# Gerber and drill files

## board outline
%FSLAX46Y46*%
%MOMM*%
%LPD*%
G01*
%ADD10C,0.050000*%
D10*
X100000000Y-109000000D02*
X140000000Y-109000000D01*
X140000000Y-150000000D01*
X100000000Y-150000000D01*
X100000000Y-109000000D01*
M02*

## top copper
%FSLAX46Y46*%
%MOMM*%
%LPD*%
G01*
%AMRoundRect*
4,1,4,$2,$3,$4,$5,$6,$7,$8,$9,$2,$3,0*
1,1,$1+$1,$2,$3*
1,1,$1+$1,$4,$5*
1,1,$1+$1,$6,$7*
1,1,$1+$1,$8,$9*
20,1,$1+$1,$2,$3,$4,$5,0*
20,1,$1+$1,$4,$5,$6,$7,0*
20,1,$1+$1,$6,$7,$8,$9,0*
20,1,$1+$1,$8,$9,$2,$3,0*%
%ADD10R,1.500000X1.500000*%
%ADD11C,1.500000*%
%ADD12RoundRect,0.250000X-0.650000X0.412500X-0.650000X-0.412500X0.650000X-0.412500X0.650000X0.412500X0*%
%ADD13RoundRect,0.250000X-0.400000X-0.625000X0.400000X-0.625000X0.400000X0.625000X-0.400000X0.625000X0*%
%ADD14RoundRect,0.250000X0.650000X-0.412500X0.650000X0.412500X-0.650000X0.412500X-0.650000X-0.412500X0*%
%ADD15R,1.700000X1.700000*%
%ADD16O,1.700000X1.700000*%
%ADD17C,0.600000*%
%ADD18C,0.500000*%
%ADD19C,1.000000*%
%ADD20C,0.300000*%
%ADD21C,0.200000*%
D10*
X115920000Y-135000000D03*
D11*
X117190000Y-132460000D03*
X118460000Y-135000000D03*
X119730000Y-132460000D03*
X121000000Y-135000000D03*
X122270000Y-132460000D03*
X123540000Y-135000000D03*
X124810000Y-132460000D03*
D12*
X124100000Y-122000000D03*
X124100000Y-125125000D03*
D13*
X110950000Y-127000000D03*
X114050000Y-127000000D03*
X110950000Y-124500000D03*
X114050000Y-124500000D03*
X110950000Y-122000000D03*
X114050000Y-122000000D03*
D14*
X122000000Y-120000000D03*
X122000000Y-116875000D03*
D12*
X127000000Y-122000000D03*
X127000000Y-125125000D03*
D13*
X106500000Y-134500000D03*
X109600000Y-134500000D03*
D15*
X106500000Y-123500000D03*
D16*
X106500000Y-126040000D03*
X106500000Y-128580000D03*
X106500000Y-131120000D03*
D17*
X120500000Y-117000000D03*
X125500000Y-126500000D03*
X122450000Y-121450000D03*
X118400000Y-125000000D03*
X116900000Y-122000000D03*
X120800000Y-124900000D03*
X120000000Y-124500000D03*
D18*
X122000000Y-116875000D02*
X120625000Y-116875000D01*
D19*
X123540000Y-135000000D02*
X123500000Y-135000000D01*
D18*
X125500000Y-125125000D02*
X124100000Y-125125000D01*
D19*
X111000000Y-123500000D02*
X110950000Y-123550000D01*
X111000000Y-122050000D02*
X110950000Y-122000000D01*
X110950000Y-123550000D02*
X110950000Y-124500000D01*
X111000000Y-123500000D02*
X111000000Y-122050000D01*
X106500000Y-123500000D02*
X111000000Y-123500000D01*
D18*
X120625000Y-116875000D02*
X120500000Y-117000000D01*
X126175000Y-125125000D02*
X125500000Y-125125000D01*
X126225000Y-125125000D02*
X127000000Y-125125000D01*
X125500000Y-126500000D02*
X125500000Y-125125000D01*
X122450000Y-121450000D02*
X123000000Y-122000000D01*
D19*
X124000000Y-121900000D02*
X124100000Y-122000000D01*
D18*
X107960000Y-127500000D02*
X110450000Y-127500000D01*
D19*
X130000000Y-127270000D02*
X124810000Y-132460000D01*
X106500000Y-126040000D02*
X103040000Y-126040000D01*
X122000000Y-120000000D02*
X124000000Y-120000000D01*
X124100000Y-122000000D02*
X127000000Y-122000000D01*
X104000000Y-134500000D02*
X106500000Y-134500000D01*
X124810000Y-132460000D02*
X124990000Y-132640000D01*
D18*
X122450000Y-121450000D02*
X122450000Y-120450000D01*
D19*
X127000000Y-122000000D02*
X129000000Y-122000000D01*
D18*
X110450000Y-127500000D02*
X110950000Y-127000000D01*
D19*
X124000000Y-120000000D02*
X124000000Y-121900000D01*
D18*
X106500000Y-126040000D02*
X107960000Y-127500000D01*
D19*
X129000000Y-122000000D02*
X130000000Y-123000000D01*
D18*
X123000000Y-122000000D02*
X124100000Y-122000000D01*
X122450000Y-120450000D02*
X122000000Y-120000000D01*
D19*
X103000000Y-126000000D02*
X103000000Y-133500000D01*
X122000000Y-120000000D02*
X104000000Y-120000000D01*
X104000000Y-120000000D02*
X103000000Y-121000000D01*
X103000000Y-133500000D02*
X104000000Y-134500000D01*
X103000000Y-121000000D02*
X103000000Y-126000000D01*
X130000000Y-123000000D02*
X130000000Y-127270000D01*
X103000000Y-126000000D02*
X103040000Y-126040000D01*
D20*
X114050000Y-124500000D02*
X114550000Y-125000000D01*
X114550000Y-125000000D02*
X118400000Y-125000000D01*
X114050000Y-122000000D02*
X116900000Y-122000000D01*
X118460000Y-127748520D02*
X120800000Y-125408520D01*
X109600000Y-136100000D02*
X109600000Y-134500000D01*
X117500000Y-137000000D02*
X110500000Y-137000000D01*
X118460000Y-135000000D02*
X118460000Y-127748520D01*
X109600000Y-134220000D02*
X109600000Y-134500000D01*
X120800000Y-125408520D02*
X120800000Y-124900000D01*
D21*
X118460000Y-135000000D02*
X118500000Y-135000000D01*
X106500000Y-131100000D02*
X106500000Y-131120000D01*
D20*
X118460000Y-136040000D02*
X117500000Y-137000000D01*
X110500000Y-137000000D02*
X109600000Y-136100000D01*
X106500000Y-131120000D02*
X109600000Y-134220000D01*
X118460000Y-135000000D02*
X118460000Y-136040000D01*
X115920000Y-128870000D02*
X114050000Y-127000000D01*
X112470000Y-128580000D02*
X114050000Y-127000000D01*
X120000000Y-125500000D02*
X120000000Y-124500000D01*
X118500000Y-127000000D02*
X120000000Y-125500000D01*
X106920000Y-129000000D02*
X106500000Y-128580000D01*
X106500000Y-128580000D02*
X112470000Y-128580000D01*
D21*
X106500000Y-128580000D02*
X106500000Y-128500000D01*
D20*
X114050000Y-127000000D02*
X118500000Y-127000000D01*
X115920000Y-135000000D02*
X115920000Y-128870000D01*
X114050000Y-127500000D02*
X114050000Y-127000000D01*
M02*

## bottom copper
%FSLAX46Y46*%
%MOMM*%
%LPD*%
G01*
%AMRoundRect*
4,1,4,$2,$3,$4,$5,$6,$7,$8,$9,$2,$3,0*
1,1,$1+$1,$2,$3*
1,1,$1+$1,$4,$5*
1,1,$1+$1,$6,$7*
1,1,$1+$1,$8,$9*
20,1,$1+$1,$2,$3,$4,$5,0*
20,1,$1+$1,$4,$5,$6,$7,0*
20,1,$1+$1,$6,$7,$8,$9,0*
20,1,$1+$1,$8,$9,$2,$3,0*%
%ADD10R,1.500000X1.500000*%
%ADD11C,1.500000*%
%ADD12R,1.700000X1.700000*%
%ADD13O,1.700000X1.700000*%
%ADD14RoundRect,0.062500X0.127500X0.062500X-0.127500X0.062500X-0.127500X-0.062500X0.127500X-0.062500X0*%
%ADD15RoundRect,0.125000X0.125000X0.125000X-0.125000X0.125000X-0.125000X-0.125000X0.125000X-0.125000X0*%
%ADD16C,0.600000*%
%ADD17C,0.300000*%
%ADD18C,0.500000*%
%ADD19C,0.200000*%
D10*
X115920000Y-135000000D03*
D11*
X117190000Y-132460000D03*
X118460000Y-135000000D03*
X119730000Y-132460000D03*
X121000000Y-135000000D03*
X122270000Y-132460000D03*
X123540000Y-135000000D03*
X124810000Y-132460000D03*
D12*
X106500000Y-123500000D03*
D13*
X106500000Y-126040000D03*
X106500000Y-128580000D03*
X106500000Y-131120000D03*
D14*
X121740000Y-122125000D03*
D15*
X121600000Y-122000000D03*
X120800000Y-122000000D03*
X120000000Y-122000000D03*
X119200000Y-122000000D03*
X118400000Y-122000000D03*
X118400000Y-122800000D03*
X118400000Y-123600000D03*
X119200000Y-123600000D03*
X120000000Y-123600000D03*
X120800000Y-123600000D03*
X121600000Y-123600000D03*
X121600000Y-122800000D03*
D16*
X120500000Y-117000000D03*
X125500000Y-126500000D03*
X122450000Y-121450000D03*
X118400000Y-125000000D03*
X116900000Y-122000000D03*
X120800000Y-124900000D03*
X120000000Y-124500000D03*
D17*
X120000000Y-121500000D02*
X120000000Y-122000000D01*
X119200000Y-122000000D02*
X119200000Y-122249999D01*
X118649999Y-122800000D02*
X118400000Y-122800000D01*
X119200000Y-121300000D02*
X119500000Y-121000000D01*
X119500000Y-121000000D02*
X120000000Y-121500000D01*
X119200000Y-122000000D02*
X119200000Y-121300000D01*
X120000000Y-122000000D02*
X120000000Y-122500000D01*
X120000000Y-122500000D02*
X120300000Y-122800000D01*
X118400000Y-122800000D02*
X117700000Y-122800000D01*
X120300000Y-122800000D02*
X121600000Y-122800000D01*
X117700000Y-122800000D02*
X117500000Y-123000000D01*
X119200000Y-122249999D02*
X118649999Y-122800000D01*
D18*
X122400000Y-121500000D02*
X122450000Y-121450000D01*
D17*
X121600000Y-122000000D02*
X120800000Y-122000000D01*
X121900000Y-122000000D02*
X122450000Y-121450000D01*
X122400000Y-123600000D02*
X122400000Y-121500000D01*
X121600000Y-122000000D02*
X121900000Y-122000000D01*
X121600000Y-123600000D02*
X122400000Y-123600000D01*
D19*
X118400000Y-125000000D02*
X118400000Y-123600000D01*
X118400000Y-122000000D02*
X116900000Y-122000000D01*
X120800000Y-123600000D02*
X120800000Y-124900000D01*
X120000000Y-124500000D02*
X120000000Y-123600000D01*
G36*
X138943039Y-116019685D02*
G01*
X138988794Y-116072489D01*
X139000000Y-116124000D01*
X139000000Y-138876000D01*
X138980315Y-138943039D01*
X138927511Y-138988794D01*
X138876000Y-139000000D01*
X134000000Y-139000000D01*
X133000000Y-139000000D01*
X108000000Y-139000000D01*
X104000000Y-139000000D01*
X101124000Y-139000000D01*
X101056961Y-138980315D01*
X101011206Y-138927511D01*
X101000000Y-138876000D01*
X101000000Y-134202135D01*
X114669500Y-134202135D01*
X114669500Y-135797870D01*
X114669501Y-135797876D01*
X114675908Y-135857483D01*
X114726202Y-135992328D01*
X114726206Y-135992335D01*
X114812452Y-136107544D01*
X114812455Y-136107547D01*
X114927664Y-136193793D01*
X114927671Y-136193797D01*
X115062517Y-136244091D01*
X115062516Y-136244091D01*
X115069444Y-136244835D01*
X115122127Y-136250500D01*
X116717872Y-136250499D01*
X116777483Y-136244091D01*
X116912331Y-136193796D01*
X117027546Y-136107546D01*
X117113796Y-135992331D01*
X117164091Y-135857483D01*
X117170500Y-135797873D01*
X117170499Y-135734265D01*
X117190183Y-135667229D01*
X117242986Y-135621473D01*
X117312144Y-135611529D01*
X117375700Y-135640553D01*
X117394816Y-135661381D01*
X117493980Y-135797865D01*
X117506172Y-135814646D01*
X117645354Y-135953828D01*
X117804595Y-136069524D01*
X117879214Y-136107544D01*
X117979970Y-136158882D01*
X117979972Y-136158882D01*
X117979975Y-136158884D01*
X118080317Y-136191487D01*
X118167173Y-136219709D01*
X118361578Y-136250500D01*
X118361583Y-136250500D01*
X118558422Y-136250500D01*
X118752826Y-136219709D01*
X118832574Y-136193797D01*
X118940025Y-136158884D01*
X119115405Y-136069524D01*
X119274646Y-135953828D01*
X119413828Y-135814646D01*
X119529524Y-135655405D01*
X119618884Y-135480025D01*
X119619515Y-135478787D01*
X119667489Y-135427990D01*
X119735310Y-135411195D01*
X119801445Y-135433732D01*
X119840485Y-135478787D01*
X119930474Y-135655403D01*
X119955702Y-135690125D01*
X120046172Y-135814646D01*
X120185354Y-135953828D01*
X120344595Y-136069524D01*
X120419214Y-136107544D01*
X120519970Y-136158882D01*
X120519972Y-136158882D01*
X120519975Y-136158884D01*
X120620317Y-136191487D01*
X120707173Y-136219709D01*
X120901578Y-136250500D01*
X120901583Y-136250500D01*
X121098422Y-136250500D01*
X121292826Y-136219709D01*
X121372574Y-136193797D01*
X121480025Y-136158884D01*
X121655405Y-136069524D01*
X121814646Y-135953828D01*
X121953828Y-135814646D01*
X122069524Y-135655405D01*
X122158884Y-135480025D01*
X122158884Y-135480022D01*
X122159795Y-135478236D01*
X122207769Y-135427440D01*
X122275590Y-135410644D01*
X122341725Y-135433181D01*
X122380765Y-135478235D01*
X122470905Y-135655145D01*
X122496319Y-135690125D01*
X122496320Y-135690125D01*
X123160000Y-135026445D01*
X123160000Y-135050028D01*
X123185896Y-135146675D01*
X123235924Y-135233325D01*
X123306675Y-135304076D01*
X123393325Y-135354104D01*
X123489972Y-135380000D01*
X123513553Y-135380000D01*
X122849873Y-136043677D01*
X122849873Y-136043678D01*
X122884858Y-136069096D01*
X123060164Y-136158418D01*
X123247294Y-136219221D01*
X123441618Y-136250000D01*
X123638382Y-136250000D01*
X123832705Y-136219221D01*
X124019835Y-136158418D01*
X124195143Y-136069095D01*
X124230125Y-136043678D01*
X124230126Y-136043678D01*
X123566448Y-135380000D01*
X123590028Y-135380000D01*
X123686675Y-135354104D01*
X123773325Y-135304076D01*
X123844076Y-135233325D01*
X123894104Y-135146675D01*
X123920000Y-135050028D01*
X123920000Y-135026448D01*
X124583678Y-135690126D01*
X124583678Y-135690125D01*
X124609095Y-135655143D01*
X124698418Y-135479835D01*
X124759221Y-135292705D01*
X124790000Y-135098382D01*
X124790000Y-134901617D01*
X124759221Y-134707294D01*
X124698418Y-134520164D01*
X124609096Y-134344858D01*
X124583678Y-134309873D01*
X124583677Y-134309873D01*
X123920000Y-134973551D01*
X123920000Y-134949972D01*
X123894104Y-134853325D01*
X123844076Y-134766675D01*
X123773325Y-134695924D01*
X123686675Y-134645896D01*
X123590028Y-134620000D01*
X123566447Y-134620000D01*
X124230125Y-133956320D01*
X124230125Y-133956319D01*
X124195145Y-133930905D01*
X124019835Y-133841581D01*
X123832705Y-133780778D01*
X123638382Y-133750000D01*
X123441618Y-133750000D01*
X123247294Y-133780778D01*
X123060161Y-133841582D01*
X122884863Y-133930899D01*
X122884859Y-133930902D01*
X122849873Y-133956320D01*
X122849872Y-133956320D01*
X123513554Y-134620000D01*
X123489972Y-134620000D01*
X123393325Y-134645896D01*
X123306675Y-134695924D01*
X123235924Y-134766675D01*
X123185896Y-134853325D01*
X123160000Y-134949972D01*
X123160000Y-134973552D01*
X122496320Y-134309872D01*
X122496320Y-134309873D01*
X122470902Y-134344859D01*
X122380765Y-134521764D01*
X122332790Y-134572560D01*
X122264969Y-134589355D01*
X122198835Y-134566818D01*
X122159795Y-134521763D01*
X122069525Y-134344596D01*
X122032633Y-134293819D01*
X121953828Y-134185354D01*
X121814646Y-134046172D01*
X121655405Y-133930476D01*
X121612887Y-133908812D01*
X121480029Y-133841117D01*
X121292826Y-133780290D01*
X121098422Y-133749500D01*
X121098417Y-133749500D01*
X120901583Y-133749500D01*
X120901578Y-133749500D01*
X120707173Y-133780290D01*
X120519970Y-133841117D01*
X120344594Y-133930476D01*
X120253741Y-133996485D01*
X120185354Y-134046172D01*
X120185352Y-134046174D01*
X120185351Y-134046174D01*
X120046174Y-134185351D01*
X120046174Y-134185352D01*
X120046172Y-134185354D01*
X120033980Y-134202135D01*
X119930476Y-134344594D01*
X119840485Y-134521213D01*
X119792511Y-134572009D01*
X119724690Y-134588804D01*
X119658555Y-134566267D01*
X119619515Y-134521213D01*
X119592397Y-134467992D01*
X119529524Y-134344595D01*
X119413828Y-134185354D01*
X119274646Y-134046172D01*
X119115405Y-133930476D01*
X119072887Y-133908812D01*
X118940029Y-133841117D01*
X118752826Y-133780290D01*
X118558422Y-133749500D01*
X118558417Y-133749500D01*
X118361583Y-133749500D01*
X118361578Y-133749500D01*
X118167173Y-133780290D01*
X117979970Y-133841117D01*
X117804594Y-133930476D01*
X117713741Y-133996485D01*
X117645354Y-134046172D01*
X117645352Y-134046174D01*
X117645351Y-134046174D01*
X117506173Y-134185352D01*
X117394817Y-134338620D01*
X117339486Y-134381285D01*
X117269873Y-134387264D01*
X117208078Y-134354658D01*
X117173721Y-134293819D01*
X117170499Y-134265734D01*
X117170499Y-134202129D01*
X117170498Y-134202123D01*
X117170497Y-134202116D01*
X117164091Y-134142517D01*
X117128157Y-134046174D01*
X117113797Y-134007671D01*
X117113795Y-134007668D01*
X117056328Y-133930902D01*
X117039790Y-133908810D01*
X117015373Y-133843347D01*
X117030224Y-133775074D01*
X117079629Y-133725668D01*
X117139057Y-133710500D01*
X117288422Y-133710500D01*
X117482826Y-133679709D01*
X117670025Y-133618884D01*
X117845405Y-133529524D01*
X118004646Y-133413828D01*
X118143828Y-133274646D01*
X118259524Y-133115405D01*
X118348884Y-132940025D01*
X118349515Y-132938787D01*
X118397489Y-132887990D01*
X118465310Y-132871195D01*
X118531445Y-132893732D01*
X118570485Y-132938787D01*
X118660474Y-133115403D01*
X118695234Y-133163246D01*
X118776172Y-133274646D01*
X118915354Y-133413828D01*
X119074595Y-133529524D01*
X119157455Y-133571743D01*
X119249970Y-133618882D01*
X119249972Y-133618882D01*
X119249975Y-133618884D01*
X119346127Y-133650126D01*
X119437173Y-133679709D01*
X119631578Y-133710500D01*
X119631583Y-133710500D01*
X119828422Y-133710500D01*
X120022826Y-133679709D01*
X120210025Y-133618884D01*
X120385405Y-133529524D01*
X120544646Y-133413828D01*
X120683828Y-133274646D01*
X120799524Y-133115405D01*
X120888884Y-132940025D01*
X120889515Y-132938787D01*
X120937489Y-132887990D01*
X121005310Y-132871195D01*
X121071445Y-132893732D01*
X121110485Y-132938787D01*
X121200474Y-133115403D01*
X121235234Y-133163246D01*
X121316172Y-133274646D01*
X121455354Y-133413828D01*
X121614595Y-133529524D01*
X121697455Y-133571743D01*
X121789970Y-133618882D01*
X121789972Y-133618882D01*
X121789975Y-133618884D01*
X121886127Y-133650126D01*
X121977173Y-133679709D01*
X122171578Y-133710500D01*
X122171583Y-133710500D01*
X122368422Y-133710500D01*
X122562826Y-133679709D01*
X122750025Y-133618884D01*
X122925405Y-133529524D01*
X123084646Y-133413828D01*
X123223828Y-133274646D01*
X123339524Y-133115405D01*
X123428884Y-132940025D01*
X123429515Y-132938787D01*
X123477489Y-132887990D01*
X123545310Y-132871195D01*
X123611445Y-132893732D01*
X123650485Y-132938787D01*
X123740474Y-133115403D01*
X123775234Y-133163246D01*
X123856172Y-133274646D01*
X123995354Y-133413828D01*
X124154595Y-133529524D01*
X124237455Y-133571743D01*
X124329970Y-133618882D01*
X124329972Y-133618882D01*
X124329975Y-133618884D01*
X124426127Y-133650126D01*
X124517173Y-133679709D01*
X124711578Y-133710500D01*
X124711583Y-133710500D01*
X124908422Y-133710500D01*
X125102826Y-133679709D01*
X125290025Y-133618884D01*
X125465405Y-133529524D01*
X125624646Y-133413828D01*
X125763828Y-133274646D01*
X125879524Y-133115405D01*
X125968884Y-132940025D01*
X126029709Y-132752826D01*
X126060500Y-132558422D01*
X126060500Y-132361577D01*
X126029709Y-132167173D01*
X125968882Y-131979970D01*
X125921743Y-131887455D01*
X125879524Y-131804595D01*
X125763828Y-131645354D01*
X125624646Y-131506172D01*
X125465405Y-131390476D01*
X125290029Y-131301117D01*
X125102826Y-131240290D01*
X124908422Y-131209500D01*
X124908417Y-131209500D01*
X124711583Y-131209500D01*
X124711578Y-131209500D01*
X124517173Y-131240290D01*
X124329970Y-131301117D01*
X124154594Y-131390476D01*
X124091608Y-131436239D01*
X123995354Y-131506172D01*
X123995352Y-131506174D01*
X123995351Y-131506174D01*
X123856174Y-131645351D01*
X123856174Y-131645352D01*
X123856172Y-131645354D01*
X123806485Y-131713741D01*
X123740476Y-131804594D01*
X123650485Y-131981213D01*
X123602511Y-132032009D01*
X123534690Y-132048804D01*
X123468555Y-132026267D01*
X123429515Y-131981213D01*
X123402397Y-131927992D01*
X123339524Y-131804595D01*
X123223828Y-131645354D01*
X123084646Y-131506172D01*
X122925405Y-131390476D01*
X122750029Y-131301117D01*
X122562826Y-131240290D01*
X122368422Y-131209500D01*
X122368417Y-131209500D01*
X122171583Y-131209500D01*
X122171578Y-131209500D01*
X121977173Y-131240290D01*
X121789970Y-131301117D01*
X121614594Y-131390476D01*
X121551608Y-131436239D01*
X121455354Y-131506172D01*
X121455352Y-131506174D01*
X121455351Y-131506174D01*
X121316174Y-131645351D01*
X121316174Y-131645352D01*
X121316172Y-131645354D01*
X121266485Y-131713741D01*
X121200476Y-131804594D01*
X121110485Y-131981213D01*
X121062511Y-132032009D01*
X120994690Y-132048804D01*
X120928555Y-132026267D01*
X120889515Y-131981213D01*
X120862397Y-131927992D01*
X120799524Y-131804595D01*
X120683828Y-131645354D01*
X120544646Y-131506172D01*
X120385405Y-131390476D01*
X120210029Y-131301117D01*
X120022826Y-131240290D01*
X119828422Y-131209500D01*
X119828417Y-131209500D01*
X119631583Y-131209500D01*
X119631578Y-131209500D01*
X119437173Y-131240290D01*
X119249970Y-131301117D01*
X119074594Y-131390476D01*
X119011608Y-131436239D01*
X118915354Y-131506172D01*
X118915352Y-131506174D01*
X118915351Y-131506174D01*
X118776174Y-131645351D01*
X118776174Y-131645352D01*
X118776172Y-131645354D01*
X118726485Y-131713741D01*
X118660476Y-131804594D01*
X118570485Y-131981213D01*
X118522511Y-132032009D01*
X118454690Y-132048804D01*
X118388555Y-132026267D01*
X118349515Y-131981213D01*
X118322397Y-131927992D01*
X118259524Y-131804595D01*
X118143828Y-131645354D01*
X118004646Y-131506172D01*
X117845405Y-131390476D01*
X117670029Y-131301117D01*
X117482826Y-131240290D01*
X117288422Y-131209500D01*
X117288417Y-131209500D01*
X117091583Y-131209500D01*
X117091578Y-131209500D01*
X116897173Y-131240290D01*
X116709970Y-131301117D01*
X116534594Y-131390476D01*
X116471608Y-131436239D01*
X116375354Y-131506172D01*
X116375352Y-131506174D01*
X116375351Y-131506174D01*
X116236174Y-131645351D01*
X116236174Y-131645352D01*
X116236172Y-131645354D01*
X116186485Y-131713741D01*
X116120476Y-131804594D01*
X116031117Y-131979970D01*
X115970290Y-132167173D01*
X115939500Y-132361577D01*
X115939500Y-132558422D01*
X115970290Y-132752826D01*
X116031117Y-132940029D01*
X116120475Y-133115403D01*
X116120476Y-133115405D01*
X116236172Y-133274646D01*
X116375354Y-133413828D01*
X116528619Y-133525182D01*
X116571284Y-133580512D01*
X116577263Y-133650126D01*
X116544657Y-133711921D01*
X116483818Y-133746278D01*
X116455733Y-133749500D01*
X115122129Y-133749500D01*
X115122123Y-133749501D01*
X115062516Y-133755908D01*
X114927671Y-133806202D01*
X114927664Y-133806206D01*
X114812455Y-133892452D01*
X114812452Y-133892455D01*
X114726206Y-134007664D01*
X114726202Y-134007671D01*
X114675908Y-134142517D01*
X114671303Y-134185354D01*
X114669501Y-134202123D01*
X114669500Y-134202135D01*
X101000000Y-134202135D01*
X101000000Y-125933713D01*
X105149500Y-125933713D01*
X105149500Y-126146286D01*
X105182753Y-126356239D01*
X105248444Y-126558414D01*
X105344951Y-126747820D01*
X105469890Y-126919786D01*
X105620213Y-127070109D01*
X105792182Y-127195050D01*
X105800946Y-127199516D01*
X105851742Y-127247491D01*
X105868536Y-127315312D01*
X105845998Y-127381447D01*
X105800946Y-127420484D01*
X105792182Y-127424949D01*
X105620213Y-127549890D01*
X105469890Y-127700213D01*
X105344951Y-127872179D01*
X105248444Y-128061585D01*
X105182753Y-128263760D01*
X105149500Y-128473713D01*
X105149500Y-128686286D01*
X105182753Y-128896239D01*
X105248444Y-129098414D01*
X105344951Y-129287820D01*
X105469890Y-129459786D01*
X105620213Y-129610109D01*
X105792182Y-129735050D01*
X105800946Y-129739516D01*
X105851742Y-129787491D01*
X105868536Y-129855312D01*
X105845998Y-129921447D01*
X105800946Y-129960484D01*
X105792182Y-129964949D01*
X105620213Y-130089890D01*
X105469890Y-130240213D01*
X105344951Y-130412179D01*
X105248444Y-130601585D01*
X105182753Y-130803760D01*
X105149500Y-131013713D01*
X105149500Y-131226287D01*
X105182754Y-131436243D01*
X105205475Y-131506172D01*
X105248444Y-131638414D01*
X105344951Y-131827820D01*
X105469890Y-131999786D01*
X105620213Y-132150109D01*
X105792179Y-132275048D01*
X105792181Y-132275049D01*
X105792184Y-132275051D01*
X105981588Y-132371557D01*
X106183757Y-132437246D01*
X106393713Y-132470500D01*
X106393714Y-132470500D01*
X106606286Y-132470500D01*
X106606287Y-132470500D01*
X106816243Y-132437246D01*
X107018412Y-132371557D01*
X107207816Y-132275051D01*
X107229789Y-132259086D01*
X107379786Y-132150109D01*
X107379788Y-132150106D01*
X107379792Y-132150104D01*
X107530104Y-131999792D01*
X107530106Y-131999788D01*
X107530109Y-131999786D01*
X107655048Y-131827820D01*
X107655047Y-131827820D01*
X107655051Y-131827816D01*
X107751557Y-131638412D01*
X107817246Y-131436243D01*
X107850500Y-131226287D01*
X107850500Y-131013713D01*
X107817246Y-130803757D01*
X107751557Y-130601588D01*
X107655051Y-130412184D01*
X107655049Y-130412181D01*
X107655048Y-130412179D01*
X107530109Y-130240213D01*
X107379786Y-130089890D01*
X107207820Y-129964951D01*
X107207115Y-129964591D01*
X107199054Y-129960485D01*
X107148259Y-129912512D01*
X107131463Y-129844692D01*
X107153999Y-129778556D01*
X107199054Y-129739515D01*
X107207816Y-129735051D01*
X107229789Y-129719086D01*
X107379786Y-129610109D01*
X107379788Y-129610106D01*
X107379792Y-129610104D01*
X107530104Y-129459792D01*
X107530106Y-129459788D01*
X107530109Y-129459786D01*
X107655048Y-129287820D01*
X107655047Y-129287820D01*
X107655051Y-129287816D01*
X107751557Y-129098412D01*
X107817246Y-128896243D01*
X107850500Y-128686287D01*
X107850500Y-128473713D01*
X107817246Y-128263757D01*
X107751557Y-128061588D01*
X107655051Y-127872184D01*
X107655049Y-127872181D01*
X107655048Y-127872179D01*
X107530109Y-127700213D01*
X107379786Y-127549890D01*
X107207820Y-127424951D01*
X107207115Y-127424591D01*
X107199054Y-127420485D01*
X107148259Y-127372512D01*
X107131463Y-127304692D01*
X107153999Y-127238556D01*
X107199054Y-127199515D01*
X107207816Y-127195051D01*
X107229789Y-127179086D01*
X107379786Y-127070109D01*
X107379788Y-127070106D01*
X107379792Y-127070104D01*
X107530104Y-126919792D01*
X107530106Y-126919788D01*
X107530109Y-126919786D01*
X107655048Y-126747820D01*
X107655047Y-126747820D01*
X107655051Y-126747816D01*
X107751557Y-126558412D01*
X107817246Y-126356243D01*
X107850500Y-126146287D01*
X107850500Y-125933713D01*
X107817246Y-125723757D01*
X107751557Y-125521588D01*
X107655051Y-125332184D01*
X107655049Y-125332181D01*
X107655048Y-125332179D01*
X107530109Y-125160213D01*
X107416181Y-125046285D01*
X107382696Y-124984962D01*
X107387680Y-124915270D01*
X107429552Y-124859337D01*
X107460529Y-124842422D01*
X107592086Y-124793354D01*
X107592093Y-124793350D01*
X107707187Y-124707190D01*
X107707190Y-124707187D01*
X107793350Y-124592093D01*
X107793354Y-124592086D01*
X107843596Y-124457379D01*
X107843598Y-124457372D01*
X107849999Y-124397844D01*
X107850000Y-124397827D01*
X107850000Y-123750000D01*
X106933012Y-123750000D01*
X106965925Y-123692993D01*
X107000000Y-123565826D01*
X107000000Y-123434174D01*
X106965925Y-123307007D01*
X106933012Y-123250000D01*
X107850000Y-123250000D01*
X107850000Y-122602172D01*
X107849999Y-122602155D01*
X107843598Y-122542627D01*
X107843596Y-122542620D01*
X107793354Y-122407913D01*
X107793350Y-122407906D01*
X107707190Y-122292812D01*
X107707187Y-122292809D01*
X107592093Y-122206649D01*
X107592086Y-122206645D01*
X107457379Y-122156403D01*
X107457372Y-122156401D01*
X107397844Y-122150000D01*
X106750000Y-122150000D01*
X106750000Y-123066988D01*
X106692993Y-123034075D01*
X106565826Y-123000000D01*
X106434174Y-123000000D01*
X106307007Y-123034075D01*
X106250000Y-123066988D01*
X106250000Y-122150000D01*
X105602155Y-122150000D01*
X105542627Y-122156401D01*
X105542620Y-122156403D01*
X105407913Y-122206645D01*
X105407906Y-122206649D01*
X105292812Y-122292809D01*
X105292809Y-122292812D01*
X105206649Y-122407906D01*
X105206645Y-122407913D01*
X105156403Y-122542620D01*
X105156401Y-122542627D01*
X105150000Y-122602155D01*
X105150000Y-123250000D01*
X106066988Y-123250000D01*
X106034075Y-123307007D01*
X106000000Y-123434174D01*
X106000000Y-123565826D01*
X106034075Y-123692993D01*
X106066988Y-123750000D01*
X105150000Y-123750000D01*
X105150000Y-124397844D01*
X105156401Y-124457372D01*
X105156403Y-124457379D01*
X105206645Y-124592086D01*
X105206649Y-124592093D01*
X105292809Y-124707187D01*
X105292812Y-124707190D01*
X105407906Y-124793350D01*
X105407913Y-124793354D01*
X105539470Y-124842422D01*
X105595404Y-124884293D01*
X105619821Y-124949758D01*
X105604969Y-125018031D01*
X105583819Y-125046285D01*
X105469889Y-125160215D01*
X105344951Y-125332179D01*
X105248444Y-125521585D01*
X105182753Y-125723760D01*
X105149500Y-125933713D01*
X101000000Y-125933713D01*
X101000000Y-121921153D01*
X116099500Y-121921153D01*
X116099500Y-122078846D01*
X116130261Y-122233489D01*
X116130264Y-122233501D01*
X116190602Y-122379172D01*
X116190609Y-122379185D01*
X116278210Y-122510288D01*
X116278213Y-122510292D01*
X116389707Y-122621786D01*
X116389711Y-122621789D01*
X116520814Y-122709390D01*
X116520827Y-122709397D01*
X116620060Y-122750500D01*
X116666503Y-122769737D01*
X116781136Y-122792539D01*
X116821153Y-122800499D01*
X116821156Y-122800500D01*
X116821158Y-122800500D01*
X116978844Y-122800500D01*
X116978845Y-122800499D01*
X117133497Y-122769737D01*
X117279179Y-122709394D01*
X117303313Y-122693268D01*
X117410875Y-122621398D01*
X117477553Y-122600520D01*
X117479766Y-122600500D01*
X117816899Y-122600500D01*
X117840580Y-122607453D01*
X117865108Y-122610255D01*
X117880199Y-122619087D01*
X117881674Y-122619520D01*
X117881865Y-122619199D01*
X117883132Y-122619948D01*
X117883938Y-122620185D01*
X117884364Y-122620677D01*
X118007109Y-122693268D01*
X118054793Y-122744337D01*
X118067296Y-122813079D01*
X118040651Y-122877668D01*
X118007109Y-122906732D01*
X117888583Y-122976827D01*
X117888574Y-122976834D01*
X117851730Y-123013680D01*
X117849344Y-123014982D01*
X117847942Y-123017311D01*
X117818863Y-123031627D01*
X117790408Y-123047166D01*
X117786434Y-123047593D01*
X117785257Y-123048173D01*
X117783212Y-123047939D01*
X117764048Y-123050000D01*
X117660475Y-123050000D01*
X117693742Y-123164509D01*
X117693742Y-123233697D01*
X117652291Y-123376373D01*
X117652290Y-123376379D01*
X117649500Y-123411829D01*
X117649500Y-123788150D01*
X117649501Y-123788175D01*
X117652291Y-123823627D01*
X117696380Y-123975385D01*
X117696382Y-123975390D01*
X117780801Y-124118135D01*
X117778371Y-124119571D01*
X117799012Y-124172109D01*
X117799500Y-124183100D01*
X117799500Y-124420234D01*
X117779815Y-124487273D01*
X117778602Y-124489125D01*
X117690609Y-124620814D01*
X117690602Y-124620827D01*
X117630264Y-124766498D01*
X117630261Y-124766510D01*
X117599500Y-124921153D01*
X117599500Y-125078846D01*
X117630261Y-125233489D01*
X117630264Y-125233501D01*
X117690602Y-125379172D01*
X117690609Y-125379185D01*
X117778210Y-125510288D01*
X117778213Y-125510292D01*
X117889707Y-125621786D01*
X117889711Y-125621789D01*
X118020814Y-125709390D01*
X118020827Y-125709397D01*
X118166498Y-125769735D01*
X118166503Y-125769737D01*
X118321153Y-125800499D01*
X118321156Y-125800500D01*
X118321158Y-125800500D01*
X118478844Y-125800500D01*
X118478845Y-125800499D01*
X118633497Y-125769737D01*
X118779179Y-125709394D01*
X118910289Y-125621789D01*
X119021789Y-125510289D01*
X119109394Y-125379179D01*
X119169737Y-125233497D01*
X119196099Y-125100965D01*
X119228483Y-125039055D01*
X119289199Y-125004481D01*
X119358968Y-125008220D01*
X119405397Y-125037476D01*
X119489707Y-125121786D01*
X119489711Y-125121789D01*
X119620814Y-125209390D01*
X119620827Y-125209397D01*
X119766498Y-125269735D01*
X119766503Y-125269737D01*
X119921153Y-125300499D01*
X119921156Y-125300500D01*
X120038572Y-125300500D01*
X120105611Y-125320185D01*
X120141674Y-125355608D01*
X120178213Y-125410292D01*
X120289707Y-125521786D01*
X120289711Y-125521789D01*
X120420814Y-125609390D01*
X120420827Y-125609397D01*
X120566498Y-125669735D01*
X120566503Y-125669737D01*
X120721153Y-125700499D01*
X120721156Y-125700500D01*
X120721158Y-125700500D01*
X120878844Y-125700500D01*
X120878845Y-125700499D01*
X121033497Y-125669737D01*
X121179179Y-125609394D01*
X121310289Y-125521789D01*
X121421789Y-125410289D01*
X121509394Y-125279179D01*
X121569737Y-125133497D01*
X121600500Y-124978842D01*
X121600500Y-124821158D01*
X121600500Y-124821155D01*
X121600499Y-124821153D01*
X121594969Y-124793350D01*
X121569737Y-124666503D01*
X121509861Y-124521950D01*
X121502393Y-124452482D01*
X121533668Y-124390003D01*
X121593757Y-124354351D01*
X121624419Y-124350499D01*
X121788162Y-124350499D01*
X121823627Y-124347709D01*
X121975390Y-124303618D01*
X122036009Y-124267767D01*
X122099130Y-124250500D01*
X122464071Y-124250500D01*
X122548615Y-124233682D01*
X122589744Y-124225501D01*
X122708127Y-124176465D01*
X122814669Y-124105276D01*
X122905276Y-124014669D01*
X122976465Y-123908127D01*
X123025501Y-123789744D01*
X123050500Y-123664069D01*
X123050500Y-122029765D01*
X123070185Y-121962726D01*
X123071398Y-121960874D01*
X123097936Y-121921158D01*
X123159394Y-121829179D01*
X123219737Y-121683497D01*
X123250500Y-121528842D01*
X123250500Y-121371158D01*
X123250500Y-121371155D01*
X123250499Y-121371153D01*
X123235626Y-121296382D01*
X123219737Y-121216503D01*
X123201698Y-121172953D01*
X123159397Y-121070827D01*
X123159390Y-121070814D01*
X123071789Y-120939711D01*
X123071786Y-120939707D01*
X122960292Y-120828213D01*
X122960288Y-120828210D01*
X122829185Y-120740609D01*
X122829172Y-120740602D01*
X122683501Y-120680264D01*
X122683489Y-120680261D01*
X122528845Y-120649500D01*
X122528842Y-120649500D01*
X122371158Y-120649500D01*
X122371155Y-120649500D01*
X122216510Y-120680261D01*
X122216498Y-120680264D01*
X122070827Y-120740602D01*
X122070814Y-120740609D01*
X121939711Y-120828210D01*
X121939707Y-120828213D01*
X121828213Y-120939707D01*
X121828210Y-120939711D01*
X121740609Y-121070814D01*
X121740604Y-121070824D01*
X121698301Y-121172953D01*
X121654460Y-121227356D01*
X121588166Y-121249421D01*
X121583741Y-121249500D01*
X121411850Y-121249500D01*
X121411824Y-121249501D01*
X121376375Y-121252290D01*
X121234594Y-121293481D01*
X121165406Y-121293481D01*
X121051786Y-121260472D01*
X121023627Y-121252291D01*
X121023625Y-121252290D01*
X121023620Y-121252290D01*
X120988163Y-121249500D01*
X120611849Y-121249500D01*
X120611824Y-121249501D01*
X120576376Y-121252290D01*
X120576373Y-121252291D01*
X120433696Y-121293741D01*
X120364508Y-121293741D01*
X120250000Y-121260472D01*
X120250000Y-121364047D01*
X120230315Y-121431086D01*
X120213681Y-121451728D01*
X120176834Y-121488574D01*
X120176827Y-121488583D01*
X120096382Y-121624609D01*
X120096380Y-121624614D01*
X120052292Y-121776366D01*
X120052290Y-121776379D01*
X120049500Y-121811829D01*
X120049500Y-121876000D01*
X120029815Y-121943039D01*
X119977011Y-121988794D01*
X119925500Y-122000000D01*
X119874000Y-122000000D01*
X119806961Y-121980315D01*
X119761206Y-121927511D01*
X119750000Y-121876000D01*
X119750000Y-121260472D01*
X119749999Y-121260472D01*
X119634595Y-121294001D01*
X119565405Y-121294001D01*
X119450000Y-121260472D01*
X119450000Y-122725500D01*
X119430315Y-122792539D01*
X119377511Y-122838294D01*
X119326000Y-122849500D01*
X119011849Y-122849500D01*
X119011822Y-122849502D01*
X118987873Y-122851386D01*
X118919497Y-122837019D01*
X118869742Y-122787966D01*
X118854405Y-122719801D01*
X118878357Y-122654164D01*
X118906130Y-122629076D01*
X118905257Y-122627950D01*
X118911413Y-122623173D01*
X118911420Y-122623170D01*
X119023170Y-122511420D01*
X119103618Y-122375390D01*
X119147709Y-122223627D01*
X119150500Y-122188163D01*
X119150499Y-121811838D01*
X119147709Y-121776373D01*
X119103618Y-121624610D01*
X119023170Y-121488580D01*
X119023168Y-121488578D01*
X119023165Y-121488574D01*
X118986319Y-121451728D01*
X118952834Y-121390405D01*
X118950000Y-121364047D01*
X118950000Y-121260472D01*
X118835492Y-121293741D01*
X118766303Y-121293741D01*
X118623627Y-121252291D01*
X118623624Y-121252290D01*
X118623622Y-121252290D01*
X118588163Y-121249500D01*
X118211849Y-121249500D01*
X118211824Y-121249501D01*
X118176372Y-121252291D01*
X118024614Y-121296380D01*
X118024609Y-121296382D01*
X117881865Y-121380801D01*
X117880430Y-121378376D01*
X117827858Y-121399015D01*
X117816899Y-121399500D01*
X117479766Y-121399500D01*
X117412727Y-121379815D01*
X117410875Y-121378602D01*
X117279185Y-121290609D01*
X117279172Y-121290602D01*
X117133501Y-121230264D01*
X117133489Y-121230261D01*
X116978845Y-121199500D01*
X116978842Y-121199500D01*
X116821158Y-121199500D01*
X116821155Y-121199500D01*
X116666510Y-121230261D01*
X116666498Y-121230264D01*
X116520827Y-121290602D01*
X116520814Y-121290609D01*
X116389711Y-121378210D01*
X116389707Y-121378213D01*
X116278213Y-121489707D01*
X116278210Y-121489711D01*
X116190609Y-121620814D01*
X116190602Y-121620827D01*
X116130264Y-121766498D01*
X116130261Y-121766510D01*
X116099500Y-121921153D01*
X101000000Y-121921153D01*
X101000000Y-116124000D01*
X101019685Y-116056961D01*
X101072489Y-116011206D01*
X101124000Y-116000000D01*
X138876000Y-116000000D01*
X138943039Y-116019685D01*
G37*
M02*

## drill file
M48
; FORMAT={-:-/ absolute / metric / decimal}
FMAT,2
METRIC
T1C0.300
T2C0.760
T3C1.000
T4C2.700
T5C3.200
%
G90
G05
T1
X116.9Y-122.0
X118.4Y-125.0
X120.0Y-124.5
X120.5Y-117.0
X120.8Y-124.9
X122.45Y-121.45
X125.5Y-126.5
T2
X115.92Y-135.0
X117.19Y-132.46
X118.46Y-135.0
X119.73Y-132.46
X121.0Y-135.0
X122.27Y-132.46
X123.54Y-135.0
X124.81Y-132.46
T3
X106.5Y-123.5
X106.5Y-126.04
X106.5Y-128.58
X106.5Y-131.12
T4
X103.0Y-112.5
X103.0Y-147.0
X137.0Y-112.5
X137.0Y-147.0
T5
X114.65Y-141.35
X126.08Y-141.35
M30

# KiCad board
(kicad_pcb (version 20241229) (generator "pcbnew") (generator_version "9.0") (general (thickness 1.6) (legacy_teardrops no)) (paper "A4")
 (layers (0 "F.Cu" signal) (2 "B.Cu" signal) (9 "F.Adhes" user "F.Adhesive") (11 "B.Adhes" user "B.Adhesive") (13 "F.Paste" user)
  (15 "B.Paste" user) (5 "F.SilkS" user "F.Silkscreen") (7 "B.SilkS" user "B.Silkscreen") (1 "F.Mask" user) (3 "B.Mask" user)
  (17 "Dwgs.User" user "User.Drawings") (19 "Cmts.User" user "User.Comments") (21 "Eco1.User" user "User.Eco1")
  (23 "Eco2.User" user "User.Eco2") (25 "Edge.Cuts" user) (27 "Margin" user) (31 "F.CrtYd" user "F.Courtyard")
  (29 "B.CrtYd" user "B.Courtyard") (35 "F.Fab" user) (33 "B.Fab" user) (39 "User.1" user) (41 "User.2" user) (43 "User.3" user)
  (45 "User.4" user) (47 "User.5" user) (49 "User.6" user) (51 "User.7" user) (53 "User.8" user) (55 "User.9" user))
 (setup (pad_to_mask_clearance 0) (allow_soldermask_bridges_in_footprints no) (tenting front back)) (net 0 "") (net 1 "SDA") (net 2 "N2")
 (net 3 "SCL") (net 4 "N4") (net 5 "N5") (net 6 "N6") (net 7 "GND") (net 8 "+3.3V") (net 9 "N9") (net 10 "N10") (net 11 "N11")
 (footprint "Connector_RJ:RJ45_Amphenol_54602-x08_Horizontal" (layer "F.Cu") (at 115.92 135)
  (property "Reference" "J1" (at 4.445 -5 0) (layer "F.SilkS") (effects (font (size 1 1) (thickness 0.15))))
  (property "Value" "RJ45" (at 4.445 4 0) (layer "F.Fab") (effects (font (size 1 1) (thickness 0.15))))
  (pad "" np_thru_hole circle (at -1.27 6.35) (size 3.2 3.2) (drill 3.2) (layers "*.Cu" "*.Mask"))
  (pad "" np_thru_hole circle (at 10.16 6.35) (size 3.2 3.2) (drill 3.2) (layers "*.Cu" "*.Mask"))
  (pad "1" thru_hole rect (at 0 0) (size 1.5 1.5) (drill 0.76) (layers "*.Cu" "*.Mask") (remove_unused_layers no) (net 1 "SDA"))
  (pad "2" thru_hole circle (at 1.27 -2.54) (size 1.5 1.5) (drill 0.76) (layers "*.Cu" "*.Mask") (remove_unused_layers no) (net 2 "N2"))
  (pad "3" thru_hole circle (at 2.54 0) (size 1.5 1.5) (drill 0.76) (layers "*.Cu" "*.Mask") (remove_unused_layers no) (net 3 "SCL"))
  (pad "4" thru_hole circle (at 3.81 -2.54) (size 1.5 1.5) (drill 0.76) (layers "*.Cu" "*.Mask") (remove_unused_layers no) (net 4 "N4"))
  (pad "5" thru_hole circle (at 5.08 0) (size 1.5 1.5) (drill 0.76) (layers "*.Cu" "*.Mask") (remove_unused_layers no) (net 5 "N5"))
  (pad "6" thru_hole circle (at 6.35 -2.54) (size 1.5 1.5) (drill 0.76) (layers "*.Cu" "*.Mask") (remove_unused_layers no) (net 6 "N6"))
  (pad "7" thru_hole circle (at 7.62 0) (size 1.5 1.5) (drill 0.76) (layers "*.Cu" "*.Mask") (remove_unused_layers no) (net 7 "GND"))
  (pad "8" thru_hole circle (at 8.89 -2.54) (size 1.5 1.5) (drill 0.76) (layers "*.Cu" "*.Mask") (remove_unused_layers no) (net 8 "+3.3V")))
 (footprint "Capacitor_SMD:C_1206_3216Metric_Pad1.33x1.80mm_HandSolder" (layer "F.Cu") (at 124.1 123.5625 -90)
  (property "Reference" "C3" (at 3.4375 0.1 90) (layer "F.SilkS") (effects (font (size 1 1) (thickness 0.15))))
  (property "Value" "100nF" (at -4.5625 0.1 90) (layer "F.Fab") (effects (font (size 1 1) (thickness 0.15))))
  (pad "1" smd roundrect (at -1.5625 0 270) (size 1.325 1.8) (layers "F.Cu" "F.Mask" "F.Paste") (roundrect_rratio 0.188679) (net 8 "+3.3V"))
  (pad "2" smd roundrect (at 1.5625 0 270) (size 1.325 1.8) (layers "F.Cu" "F.Mask" "F.Paste") (roundrect_rratio 0.188679) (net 7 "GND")))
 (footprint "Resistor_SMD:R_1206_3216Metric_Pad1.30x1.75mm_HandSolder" (layer "F.Cu") (at 112.5 127)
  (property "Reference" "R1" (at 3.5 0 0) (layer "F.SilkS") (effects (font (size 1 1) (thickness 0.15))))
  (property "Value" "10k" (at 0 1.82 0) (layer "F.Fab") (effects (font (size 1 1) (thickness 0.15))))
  (pad "1" smd roundrect (at -1.55 0) (size 1.3 1.75) (layers "F.Cu" "F.Mask" "F.Paste") (roundrect_rratio 0.192308) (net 8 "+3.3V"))
  (pad "2" smd roundrect (at 1.55 0) (size 1.3 1.75) (layers "F.Cu" "F.Mask" "F.Paste") (roundrect_rratio 0.192308) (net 1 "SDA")))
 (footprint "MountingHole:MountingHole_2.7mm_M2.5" (layer "F.Cu") (at 137 147)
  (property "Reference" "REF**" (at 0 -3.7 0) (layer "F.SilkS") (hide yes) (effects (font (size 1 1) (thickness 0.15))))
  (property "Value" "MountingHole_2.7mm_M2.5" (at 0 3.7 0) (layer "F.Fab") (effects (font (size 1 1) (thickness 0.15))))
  (pad "" np_thru_hole circle (at 0 0) (size 2.7 2.7) (drill 2.7) (layers "*.Cu" "*.Mask")))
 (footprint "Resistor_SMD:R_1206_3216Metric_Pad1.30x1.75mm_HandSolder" (layer "F.Cu") (at 112.5 124.5)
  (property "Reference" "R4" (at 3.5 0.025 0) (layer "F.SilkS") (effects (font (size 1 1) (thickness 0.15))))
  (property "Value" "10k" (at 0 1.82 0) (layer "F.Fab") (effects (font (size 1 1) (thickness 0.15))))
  (pad "1" smd roundrect (at -1.55 0) (size 1.3 1.75) (layers "F.Cu" "F.Mask" "F.Paste") (roundrect_rratio 0.192308) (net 7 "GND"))
  (pad "2" smd roundrect (at 1.55 0) (size 1.3 1.75) (layers "F.Cu" "F.Mask" "F.Paste") (roundrect_rratio 0.192308) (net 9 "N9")))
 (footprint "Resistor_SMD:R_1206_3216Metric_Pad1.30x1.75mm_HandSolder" (layer "F.Cu") (at 112.5 122)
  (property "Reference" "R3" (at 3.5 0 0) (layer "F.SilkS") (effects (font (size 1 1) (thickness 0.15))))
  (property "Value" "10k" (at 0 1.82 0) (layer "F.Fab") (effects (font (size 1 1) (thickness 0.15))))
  (pad "1" smd roundrect (at -1.55 0) (size 1.3 1.75) (layers "F.Cu" "F.Mask" "F.Paste") (roundrect_rratio 0.192308) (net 7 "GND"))
  (pad "2" smd roundrect (at 1.55 0) (size 1.3 1.75) (layers "F.Cu" "F.Mask" "F.Paste") (roundrect_rratio 0.192308) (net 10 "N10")))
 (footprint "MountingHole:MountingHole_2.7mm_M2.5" (layer "F.Cu") (at 103 147)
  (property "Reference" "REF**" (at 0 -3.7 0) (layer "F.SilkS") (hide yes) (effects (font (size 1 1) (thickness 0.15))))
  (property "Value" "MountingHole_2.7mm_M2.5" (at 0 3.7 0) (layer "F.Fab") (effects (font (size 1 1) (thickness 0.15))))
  (pad "" np_thru_hole circle (at 0 0) (size 2.7 2.7) (drill 2.7) (layers "*.Cu" "*.Mask")))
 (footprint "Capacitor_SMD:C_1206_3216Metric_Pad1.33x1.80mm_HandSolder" (layer "F.Cu") (at 122 118.4375 90)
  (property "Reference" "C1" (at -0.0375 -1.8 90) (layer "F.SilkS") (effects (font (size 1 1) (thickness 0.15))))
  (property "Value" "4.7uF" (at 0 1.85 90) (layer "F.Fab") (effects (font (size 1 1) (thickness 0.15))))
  (pad "1" smd roundrect (at -1.5625 0 90) (size 1.325 1.8) (layers "F.Cu" "F.Mask" "F.Paste") (roundrect_rratio 0.188679) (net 8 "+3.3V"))
  (pad "2" smd roundrect (at 1.5625 0 90) (size 1.325 1.8) (layers "F.Cu" "F.Mask" "F.Paste") (roundrect_rratio 0.188679) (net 7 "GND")))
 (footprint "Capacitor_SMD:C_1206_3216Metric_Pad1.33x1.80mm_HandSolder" (layer "F.Cu") (at 127 123.5625 -90)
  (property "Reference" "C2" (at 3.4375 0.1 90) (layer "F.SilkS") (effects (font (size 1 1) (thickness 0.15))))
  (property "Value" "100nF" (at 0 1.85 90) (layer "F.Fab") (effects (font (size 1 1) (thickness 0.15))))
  (pad "1" smd roundrect (at -1.5625 0 270) (size 1.325 1.8) (layers "F.Cu" "F.Mask" "F.Paste") (roundrect_rratio 0.188679) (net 8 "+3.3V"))
  (pad "2" smd roundrect (at 1.5625 0 270) (size 1.325 1.8) (layers "F.Cu" "F.Mask" "F.Paste") (roundrect_rratio 0.188679) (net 7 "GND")))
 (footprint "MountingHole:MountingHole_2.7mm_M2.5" (layer "F.Cu") (at 103 112.5)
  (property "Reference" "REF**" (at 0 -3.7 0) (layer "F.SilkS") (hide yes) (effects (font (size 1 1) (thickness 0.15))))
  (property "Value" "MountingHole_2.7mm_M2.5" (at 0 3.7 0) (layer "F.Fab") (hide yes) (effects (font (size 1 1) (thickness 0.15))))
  (pad "" np_thru_hole circle (at 0 0) (size 2.7 2.7) (drill 2.7) (layers "*.Cu" "*.Mask")))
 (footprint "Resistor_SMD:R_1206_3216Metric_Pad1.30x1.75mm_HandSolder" (layer "F.Cu") (at 108.05 134.5)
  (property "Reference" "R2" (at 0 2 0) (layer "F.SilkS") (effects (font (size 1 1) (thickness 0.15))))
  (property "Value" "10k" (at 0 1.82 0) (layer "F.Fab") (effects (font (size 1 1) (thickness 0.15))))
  (pad "1" smd roundrect (at -1.55 0) (size 1.3 1.75) (layers "F.Cu" "F.Mask" "F.Paste") (roundrect_rratio 0.192308) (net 8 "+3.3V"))
  (pad "2" smd roundrect (at 1.55 0) (size 1.3 1.75) (layers "F.Cu" "F.Mask" "F.Paste") (roundrect_rratio 0.192308) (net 3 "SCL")))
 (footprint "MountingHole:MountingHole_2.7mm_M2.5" (layer "F.Cu") (at 137 112.5)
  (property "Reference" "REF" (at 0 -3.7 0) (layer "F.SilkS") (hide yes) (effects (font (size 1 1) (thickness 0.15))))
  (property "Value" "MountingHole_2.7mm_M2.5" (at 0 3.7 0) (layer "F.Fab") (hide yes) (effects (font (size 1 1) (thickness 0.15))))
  (pad "" np_thru_hole circle (at 0 0) (size 2.7 2.7) (drill 2.7) (layers "*.Cu" "*.Mask")))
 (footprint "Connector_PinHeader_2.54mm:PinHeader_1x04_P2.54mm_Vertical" (layer "F.Cu") (at 106.5 123.5)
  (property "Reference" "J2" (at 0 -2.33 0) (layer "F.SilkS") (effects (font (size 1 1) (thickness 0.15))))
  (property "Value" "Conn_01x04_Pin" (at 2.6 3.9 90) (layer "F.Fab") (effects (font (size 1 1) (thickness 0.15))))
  (pad "1" thru_hole rect (at 0 0) (size 1.7 1.7) (drill 1) (layers "*.Cu" "*.Mask") (remove_unused_layers no) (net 7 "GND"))
  (pad "2" thru_hole oval (at 0 2.54) (size 1.7 1.7) (drill 1) (layers "*.Cu" "*.Mask") (remove_unused_layers no) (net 8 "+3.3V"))
  (pad "3" thru_hole oval (at 0 5.08) (size 1.7 1.7) (drill 1) (layers "*.Cu" "*.Mask") (remove_unused_layers no) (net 1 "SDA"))
  (pad "4" thru_hole oval (at 0 7.62) (size 1.7 1.7) (drill 1) (layers "*.Cu" "*.Mask") (remove_unused_layers no) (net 3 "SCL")))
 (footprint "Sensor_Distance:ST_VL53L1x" (layer "B.Cu") (at 120 122.8 180)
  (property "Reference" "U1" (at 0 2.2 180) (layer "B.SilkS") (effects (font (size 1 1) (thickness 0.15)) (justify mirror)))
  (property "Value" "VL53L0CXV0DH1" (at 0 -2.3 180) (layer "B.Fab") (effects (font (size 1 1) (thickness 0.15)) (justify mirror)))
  (pad "1" smd roundrect (at -1.74 0.675 180) (size 0.38 0.25) (layers "B.Cu" "B.Mask" "B.Paste") (roundrect_rratio 0.25) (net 8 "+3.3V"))
  (pad "1" smd roundrect (at -1.6 0.8 180) (size 0.5 0.5) (layers "B.Cu" "B.Mask" "B.Paste") (roundrect_rratio 0.25) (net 8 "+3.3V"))
  (pad "2" smd roundrect (at -0.8 0.8 180) (size 0.5 0.5) (layers "B.Cu" "B.Mask" "B.Paste") (roundrect_rratio 0.25) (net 8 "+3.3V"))
  (pad "3" smd roundrect (at 0 0.8 180) (size 0.5 0.5) (layers "B.Cu" "B.Mask" "B.Paste") (roundrect_rratio 0.25) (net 7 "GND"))
  (pad "4" smd roundrect (at 0.8 0.8 180) (size 0.5 0.5) (layers "B.Cu" "B.Mask" "B.Paste") (roundrect_rratio 0.25) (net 7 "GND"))
  (pad "5" smd roundrect (at 1.6 0.8 180) (size 0.5 0.5) (layers "B.Cu" "B.Mask" "B.Paste") (roundrect_rratio 0.25) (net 10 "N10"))
  (pad "6" smd roundrect (at 1.6 0 180) (size 0.5 0.5) (layers "B.Cu" "B.Mask" "B.Paste") (roundrect_rratio 0.25) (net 7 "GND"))
  (pad "7" smd roundrect (at 1.6 -0.8 180) (size 0.5 0.5) (layers "B.Cu" "B.Mask" "B.Paste") (roundrect_rratio 0.25) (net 9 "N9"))
  (pad "8" smd roundrect (at 0.8 -0.8 180) (size 0.5 0.5) (layers "B.Cu" "B.Mask" "B.Paste") (roundrect_rratio 0.25) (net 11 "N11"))
  (pad "9" smd roundrect (at 0 -0.8 180) (size 0.5 0.5) (layers "B.Cu" "B.Mask" "B.Paste") (roundrect_rratio 0.25) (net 1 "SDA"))
  (pad "10" smd roundrect (at -0.8 -0.8 180) (size 0.5 0.5) (layers "B.Cu" "B.Mask" "B.Paste") (roundrect_rratio 0.25) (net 3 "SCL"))
  (pad "11" smd roundrect (at -1.6 -0.8 180) (size 0.5 0.5) (layers "B.Cu" "B.Mask" "B.Paste") (roundrect_rratio 0.25) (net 8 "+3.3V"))
  (pad "12" smd roundrect (at -1.6 0 180) (size 0.5 0.5) (layers "B.Cu" "B.Mask" "B.Paste") (roundrect_rratio 0.25) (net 7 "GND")))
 (gr_rect (start 100 109) (end 140 150) (stroke (width 0.05) (type default)) (fill no) (layer "Edge.Cuts"))
 (segment (start 122 116.875) (end 120.625 116.875) (width 0.5) (layer "F.Cu") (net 7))
 (segment (start 123.54 135) (end 123.5 135) (width 1) (layer "F.Cu") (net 7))
 (segment (start 125.5 125.125) (end 124.1 125.125) (width 0.5) (layer "F.Cu") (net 7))
 (segment (start 111 123.5) (end 110.95 123.55) (width 1) (layer "F.Cu") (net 7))
 (segment (start 111 122.05) (end 110.95 122) (width 1) (layer "F.Cu") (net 7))
 (segment (start 110.95 123.55) (end 110.95 124.5) (width 1) (layer "F.Cu") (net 7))
 (segment (start 111 123.5) (end 111 122.05) (width 1) (layer "F.Cu") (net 7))
 (segment (start 106.5 123.5) (end 111 123.5) (width 1) (layer "F.Cu") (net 7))
 (segment (start 120.625 116.875) (end 120.5 117) (width 0.5) (layer "F.Cu") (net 7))
 (segment (start 126.175 125.125) (end 125.5 125.125) (width 0.5) (layer "F.Cu") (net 7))
 (segment (start 126.225 125.125) (end 127 125.125) (width 0.5) (layer "F.Cu") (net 7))
 (segment (start 125.5 126.5) (end 125.5 125.125) (width 0.5) (layer "F.Cu") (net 7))
 (via (at 120.5 117) (size 0.6) (drill 0.3) (layers "F.Cu" "B.Cu") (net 7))
 (via (at 125.5 126.5) (size 0.6) (drill 0.3) (layers "F.Cu" "B.Cu") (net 7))
 (segment (start 120 121.5) (end 120 122) (width 0.3) (layer "B.Cu") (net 7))
 (segment (start 119.2 122) (end 119.2 122.249999) (width 0.3) (layer "B.Cu") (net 7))
 (segment (start 118.649999 122.8) (end 118.4 122.8) (width 0.3) (layer "B.Cu") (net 7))
 (segment (start 119.2 121.3) (end 119.5 121) (width 0.3) (layer "B.Cu") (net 7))
 (segment (start 119.5 121) (end 120 121.5) (width 0.3) (layer "B.Cu") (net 7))
 (segment (start 119.2 122) (end 119.2 121.3) (width 0.3) (layer "B.Cu") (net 7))
 (segment (start 120 122) (end 120 122.5) (width 0.3) (layer "B.Cu") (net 7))
 (segment (start 120 122.5) (end 120.3 122.8) (width 0.3) (layer "B.Cu") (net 7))
 (segment (start 118.4 122.8) (end 117.7 122.8) (width 0.3) (layer "B.Cu") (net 7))
 (segment (start 120.3 122.8) (end 121.6 122.8) (width 0.3) (layer "B.Cu") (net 7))
 (segment (start 117.7 122.8) (end 117.5 123) (width 0.3) (layer "B.Cu") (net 7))
 (segment (start 119.2 122.249999) (end 118.649999 122.8) (width 0.3) (layer "B.Cu") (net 7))
 (segment (start 122.45 121.45) (end 123 122) (width 0.5) (layer "F.Cu") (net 8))
 (segment (start 124 121.9) (end 124.1 122) (width 1) (layer "F.Cu") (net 8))
 (segment (start 107.96 127.5) (end 110.45 127.5) (width 0.5) (layer "F.Cu") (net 8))
 (segment (start 130 127.27) (end 124.81 132.46) (width 1) (layer "F.Cu") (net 8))
 (segment (start 106.5 126.04) (end 103.04 126.04) (width 1) (layer "F.Cu") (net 8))
 (segment (start 122 120) (end 124 120) (width 1) (layer "F.Cu") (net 8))
 (segment (start 124.1 122) (end 127 122) (width 1) (layer "F.Cu") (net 8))
 (segment (start 104 134.5) (end 106.5 134.5) (width 1) (layer "F.Cu") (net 8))
 (segment (start 124.81 132.46) (end 124.99 132.64) (width 1) (layer "F.Cu") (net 8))
 (segment (start 122.45 121.45) (end 122.45 120.45) (width 0.5) (layer "F.Cu") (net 8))
 (segment (start 127 122) (end 129 122) (width 1) (layer "F.Cu") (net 8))
 (segment (start 110.45 127.5) (end 110.95 127) (width 0.5) (layer "F.Cu") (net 8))
 (segment (start 124 120) (end 124 121.9) (width 1) (layer "F.Cu") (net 8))
 (segment (start 106.5 126.04) (end 107.96 127.5) (width 0.5) (layer "F.Cu") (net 8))
 (segment (start 129 122) (end 130 123) (width 1) (layer "F.Cu") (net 8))
 (segment (start 123 122) (end 124.1 122) (width 0.5) (layer "F.Cu") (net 8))
 (segment (start 122.45 120.45) (end 122 120) (width 0.5) (layer "F.Cu") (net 8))
 (segment (start 103 126) (end 103 133.5) (width 1) (layer "F.Cu") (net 8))
 (segment (start 122 120) (end 104 120) (width 1) (layer "F.Cu") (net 8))
 (segment (start 104 120) (end 103 121) (width 1) (layer "F.Cu") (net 8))
 (segment (start 103 133.5) (end 104 134.5) (width 1) (layer "F.Cu") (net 8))
 (segment (start 103 121) (end 103 126) (width 1) (layer "F.Cu") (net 8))
 (segment (start 130 123) (end 130 127.27) (width 1) (layer "F.Cu") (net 8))
 (segment (start 103 126) (end 103.04 126.04) (width 1) (layer "F.Cu") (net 8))
 (via (at 122.45 121.45) (size 0.6) (drill 0.3) (layers "F.Cu" "B.Cu") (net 8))
 (segment (start 122.4 121.5) (end 122.45 121.45) (width 0.5) (layer "B.Cu") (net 8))
 (segment (start 121.6 122) (end 120.8 122) (width 0.3) (layer "B.Cu") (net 8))
 (segment (start 121.9 122) (end 122.45 121.45) (width 0.3) (layer "B.Cu") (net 8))
 (segment (start 122.4 123.6) (end 122.4 121.5) (width 0.3) (layer "B.Cu") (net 8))
 (segment (start 121.6 122) (end 121.9 122) (width 0.3) (layer "B.Cu") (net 8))
 (segment (start 121.6 123.6) (end 122.4 123.6) (width 0.3) (layer "B.Cu") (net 8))
 (segment (start 114.05 124.5) (end 114.55 125) (width 0.3) (layer "F.Cu") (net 9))
 (segment (start 114.55 125) (end 118.4 125) (width 0.3) (layer "F.Cu") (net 9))
 (via (at 118.4 125) (size 0.6) (drill 0.3) (layers "F.Cu" "B.Cu") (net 9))
 (segment (start 118.4 125) (end 118.4 123.6) (width 0.2) (layer "B.Cu") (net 9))
 (segment (start 114.05 122) (end 116.9 122) (width 0.3) (layer "F.Cu") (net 10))
 (via (at 116.9 122) (size 0.6) (drill 0.3) (layers "F.Cu" "B.Cu") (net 10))
 (segment (start 118.4 122) (end 116.9 122) (width 0.2) (layer "B.Cu") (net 10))
 (segment (start 118.46 127.74852) (end 120.8 125.40852) (width 0.3) (layer "F.Cu") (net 3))
 (segment (start 109.6 136.1) (end 109.6 134.5) (width 0.3) (layer "F.Cu") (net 3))
 (segment (start 117.5 137) (end 110.5 137) (width 0.3) (layer "F.Cu") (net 3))
 (segment (start 118.46 135) (end 118.46 127.74852) (width 0.3) (layer "F.Cu") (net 3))
 (segment (start 109.6 134.22) (end 109.6 134.5) (width 0.3) (layer "F.Cu") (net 3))
 (segment (start 120.8 125.40852) (end 120.8 124.9) (width 0.3) (layer "F.Cu") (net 3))
 (segment (start 118.46 135) (end 118.5 135) (width 0.2) (layer "F.Cu") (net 3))
 (segment (start 106.5 131.1) (end 106.5 131.12) (width 0.2) (layer "F.Cu") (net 3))
 (segment (start 118.46 136.04) (end 117.5 137) (width 0.3) (layer "F.Cu") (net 3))
 (segment (start 110.5 137) (end 109.6 136.1) (width 0.3) (layer "F.Cu") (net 3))
 (segment (start 106.5 131.12) (end 109.6 134.22) (width 0.3) (layer "F.Cu") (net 3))
 (segment (start 118.46 135) (end 118.46 136.04) (width 0.3) (layer "F.Cu") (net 3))
 (via (at 120.8 124.9) (size 0.6) (drill 0.3) (layers "F.Cu" "B.Cu") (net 3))
 (segment (start 120.8 123.6) (end 120.8 124.9) (width 0.2) (layer "B.Cu") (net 3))
 (segment (start 115.92 128.87) (end 114.05 127) (width 0.3) (layer "F.Cu") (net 1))
 (segment (start 112.47 128.58) (end 114.05 127) (width 0.3) (layer "F.Cu") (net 1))
 (segment (start 120 125.5) (end 120 124.5) (width 0.3) (layer "F.Cu") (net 1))
 (segment (start 118.5 127) (end 120 125.5) (width 0.3) (layer "F.Cu") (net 1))
 (segment (start 106.92 129) (end 106.5 128.58) (width 0.3) (layer "F.Cu") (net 1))
 (segment (start 106.5 128.58) (end 112.47 128.58) (width 0.3) (layer "F.Cu") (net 1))
 (segment (start 106.5 128.58) (end 106.5 128.5) (width 0.2) (layer "F.Cu") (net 1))
 (segment (start 114.05 127) (end 118.5 127) (width 0.3) (layer "F.Cu") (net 1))
 (segment (start 115.92 135) (end 115.92 128.87) (width 0.3) (layer "F.Cu") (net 1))
 (segment (start 114.05 127.5) (end 114.05 127) (width 0.3) (layer "F.Cu") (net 1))
 (via (at 120 124.5) (size 0.6) (drill 0.3) (layers "F.Cu" "B.Cu") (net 1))
 (segment (start 120 124.5) (end 120 123.6) (width 0.2) (layer "B.Cu") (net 1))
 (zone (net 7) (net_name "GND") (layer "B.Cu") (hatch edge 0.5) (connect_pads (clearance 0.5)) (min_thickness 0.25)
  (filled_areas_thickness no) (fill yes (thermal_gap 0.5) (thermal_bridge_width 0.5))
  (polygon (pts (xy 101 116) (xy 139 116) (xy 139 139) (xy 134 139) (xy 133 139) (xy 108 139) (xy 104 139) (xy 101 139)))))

